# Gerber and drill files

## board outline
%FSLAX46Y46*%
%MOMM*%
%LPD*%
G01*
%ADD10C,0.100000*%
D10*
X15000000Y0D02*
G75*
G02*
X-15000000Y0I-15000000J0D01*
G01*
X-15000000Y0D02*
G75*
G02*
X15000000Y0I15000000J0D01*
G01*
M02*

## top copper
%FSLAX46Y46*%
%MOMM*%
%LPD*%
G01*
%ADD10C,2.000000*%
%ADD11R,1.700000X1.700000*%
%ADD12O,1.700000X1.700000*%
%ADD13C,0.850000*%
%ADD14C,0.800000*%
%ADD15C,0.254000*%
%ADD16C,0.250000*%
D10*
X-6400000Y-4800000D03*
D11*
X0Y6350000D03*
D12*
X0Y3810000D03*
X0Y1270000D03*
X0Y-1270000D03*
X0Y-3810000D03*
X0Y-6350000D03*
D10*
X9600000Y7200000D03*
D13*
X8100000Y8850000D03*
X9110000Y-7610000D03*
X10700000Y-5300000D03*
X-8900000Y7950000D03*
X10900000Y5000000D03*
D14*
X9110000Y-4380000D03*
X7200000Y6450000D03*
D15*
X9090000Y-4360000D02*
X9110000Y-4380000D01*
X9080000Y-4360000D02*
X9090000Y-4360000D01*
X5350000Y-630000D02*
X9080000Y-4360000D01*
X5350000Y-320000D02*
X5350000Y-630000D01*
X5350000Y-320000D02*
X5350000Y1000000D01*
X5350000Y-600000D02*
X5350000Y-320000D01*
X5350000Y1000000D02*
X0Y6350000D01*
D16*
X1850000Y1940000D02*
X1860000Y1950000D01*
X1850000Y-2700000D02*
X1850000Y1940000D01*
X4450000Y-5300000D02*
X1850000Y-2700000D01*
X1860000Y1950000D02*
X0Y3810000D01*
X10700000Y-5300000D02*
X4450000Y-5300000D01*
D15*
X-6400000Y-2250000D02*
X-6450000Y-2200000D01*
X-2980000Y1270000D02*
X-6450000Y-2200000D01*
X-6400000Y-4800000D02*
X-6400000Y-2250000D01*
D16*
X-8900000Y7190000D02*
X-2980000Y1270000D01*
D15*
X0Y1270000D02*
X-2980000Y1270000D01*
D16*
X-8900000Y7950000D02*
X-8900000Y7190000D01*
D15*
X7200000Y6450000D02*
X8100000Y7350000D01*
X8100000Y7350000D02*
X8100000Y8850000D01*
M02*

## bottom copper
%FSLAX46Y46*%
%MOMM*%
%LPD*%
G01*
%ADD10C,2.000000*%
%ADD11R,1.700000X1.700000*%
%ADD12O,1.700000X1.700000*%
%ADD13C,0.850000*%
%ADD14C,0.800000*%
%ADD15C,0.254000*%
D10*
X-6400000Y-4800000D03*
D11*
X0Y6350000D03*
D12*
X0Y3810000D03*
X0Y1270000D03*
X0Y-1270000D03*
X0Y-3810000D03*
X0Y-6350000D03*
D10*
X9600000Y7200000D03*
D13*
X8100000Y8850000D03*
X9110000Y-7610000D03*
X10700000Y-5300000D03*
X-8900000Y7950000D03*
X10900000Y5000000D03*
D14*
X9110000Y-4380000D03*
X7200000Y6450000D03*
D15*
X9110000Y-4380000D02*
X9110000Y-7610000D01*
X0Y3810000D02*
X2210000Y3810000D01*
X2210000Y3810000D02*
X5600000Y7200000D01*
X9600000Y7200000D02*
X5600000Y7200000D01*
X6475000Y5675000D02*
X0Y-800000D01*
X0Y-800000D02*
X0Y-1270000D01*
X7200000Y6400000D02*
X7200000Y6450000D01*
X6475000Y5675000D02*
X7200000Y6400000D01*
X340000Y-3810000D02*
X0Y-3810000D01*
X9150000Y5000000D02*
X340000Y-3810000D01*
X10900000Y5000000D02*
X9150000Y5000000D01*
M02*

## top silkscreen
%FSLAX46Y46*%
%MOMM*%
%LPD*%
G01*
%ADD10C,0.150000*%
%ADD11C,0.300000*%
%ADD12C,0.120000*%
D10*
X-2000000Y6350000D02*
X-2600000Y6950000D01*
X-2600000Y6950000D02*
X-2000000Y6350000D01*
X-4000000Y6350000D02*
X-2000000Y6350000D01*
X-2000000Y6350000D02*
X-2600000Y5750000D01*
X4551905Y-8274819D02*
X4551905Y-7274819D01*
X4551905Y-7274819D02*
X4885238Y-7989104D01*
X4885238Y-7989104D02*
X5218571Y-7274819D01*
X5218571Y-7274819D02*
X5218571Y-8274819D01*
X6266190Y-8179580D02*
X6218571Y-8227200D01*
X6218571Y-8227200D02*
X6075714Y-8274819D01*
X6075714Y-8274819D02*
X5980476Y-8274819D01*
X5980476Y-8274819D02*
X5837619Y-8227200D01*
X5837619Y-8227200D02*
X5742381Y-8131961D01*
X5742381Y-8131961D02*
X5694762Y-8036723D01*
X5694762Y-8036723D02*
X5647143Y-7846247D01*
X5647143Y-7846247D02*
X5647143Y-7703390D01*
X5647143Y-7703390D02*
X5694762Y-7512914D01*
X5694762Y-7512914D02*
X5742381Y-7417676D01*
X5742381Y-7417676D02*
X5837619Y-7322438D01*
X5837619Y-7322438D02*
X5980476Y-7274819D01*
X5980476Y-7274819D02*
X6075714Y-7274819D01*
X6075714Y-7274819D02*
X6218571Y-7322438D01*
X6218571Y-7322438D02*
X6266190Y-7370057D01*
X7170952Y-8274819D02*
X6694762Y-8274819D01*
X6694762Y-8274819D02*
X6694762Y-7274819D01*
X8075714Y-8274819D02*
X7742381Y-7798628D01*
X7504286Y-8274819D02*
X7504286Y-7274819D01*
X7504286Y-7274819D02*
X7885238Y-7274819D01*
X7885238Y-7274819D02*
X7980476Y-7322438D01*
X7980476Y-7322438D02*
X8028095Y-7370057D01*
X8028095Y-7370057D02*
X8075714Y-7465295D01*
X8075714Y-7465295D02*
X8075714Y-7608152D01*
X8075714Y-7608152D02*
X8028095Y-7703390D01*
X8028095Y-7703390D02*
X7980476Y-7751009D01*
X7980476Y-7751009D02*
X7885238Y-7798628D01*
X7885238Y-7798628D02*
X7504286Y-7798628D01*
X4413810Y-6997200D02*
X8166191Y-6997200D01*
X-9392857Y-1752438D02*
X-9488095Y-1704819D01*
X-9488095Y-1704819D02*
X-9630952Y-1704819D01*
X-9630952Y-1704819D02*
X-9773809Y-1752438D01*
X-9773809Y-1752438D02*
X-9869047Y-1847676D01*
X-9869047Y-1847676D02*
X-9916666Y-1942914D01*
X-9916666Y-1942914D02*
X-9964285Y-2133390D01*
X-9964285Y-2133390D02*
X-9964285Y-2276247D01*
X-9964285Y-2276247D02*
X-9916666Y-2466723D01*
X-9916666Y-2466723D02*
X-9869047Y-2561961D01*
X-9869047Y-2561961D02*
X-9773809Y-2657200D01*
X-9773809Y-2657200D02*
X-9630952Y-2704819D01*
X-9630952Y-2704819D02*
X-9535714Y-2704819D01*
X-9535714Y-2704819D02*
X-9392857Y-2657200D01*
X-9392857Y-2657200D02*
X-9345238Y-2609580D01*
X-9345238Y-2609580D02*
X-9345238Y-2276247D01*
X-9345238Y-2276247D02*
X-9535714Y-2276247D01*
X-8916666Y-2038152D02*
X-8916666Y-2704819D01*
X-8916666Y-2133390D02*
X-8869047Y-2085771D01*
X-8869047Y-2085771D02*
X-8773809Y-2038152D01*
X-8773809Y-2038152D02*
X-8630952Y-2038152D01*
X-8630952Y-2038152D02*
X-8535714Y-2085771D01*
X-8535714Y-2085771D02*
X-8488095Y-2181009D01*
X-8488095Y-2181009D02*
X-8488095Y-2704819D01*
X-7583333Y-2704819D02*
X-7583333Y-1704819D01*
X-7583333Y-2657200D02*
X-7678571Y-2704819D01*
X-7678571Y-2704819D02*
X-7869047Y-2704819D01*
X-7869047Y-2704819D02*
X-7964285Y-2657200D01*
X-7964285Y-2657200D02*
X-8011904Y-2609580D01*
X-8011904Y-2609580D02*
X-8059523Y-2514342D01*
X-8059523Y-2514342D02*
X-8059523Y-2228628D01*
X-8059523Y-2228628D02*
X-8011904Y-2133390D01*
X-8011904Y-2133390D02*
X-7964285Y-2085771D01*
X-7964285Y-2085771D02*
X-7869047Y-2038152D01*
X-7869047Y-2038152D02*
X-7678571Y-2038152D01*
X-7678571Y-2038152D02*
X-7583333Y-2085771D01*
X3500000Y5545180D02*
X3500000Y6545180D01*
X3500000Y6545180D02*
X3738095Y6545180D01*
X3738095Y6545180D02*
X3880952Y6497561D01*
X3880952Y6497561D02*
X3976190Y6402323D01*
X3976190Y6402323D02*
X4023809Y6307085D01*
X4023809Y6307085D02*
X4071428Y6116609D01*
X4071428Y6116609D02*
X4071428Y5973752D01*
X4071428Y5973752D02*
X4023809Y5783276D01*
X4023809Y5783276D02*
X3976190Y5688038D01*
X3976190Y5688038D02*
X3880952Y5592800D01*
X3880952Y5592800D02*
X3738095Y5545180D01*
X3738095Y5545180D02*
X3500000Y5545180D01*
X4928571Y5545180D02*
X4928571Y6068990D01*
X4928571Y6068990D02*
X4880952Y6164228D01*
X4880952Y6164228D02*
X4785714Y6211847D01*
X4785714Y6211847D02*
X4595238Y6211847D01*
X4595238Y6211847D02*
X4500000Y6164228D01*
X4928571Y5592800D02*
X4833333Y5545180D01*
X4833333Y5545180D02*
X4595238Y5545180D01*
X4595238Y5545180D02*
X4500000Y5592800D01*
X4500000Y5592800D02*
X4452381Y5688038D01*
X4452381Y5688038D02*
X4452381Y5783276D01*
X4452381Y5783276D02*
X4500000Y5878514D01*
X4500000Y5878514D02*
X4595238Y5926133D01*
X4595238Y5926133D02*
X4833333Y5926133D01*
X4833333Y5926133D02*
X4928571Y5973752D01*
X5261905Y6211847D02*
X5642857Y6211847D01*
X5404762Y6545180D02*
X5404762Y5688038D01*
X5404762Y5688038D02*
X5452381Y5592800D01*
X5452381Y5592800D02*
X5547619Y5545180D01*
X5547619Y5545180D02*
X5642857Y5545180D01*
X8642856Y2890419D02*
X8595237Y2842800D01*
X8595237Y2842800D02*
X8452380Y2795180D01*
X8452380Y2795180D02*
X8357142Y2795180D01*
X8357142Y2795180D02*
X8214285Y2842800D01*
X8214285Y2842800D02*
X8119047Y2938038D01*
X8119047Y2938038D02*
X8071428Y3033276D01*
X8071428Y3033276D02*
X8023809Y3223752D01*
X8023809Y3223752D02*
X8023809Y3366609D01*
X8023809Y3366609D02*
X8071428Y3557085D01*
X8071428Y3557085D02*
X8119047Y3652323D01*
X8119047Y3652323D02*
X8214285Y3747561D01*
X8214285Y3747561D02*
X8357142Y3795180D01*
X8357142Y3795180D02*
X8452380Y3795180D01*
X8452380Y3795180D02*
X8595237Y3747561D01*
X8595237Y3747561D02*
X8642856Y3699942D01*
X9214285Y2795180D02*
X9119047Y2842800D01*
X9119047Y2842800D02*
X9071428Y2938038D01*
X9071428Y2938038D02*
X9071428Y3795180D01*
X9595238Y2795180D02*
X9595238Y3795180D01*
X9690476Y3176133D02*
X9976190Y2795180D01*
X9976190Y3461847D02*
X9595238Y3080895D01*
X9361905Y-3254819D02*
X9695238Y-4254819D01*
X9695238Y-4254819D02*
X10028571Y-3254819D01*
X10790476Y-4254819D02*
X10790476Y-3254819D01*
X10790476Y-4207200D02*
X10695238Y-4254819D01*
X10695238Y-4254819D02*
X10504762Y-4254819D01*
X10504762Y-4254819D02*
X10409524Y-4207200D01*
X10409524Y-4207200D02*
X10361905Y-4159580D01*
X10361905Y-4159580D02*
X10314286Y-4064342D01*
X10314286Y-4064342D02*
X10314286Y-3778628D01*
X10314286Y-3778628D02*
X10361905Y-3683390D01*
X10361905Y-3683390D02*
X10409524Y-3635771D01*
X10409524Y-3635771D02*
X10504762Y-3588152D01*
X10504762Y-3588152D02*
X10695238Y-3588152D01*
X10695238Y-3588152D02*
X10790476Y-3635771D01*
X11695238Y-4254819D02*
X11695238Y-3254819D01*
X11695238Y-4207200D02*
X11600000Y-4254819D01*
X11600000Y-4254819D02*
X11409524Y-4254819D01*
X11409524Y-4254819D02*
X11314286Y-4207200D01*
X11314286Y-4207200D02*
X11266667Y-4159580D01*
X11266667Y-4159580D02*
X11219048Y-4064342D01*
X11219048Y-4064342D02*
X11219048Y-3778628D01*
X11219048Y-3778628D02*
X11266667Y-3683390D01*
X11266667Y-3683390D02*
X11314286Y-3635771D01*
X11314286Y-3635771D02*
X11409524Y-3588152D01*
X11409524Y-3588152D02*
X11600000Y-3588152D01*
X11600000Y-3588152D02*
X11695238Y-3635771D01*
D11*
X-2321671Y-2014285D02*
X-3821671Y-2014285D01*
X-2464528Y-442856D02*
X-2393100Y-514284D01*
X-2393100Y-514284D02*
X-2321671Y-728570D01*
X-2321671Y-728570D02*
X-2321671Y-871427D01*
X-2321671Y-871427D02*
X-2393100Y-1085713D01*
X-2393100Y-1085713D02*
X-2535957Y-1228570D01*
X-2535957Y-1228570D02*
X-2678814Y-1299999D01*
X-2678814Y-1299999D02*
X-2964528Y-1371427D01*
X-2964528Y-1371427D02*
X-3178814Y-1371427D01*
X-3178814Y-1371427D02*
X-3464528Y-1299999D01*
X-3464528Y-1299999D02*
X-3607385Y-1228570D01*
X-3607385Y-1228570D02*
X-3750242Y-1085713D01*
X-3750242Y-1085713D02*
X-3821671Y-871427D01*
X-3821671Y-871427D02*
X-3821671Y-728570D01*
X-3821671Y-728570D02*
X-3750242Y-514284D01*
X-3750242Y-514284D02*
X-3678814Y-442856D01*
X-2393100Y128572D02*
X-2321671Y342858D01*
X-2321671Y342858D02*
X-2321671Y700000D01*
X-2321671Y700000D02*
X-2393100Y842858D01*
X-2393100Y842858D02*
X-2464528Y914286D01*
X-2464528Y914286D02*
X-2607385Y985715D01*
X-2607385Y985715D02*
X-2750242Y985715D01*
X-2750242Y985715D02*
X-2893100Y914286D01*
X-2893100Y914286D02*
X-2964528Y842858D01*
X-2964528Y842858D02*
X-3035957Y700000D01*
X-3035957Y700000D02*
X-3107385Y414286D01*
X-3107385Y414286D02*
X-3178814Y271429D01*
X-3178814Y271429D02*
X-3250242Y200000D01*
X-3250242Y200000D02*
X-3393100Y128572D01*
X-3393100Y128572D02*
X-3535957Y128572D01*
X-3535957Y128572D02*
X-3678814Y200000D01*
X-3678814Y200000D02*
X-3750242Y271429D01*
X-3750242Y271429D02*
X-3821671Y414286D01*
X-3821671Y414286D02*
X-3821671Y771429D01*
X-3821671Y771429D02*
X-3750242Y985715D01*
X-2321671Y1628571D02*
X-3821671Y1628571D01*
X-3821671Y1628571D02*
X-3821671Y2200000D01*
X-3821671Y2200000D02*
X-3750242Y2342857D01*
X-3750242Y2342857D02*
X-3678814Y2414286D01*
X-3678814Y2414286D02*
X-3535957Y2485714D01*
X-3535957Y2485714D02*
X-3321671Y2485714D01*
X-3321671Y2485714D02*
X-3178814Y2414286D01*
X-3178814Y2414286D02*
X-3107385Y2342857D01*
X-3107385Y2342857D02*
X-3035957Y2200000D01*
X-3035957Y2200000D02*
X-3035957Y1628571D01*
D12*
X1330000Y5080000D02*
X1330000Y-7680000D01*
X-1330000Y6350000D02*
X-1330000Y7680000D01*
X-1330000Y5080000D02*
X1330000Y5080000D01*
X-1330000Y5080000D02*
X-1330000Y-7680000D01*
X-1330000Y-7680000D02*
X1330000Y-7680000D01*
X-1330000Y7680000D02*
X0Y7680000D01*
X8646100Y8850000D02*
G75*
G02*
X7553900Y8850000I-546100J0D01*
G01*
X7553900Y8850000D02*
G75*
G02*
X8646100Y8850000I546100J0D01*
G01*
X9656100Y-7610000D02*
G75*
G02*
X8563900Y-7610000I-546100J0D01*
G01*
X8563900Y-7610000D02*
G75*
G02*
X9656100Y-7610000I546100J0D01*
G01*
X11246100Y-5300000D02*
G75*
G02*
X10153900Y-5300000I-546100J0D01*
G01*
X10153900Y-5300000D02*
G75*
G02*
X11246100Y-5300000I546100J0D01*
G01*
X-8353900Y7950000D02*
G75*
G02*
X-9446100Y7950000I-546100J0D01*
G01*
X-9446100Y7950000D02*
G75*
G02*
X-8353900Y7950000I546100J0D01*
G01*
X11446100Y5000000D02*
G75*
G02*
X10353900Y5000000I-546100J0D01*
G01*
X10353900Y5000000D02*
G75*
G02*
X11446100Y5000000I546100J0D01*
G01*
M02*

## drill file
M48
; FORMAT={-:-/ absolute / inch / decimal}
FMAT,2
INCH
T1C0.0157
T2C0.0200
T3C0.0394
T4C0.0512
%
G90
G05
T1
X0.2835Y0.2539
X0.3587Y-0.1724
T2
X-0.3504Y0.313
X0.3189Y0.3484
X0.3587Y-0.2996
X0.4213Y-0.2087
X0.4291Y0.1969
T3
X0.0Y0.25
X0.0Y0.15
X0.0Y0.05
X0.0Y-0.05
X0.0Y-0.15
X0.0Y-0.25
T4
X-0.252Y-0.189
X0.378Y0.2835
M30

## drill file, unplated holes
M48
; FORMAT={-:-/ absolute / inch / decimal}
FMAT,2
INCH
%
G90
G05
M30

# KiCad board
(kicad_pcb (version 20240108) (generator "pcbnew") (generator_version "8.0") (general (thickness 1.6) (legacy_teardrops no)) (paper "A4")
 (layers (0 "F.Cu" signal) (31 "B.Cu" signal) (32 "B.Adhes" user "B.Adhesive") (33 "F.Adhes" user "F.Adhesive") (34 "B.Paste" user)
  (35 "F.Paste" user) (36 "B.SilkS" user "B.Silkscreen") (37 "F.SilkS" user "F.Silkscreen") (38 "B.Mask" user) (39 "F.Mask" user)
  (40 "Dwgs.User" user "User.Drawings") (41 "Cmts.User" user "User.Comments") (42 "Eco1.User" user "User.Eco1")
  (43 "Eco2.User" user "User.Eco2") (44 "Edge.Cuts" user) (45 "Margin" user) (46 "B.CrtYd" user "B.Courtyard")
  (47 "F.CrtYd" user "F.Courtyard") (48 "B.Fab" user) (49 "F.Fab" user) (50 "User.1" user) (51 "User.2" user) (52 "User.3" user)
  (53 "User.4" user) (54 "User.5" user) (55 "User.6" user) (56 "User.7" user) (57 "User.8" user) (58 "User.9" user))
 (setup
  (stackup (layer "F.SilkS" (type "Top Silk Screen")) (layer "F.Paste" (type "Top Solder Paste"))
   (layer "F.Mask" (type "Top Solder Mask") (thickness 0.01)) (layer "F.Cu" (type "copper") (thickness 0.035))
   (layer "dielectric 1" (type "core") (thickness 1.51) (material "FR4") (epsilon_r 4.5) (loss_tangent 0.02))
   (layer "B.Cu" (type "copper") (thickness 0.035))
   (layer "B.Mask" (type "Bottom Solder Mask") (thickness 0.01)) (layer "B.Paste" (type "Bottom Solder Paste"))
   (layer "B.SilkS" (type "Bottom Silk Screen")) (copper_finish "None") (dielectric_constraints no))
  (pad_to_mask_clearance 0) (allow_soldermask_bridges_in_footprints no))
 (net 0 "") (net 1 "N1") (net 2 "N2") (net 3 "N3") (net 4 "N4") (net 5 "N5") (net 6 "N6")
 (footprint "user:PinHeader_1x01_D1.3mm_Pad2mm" (layer "F.Cu") (at -6.4 4.8)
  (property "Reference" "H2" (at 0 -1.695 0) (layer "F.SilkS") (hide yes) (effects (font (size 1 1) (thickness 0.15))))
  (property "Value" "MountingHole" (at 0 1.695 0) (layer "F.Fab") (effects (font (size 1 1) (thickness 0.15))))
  (pad "1" thru_hole circle (at 0 0) (size 2 2) (drill 1.3) (layers "*.Cu" "*.Mask") (remove_unused_layers no) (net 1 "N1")))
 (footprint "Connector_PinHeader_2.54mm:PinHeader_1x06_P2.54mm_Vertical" (layer "F.Cu") (at 0 -6.35)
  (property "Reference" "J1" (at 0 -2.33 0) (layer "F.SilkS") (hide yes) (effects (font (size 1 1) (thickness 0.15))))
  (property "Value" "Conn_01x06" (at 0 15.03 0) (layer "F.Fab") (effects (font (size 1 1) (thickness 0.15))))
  (fp_line (start -1.33 -1.33) (end 0 -1.33) (stroke (width 0.12) (type solid)) (layer "F.SilkS"))
  (fp_line (start -1.33 0) (end -1.33 -1.33) (stroke (width 0.12) (type solid)) (layer "F.SilkS"))
  (fp_line (start -1.33 1.27) (end -1.33 14.03) (stroke (width 0.12) (type solid)) (layer "F.SilkS"))
  (fp_line (start -1.33 1.27) (end 1.33 1.27) (stroke (width 0.12) (type solid)) (layer "F.SilkS"))
  (fp_line (start -1.33 14.03) (end 1.33 14.03) (stroke (width 0.12) (type solid)) (layer "F.SilkS"))
  (fp_line (start 1.33 1.27) (end 1.33 14.03) (stroke (width 0.12) (type solid)) (layer "F.SilkS"))
  (pad "1" thru_hole rect (at 0 0) (size 1.7 1.7) (drill 1) (layers "*.Cu" "*.Mask") (remove_unused_layers no) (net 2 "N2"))
  (pad "2" thru_hole oval (at 0 2.54) (size 1.7 1.7) (drill 1) (layers "*.Cu" "*.Mask") (remove_unused_layers no) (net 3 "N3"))
  (pad "3" thru_hole oval (at 0 5.08) (size 1.7 1.7) (drill 1) (layers "*.Cu" "*.Mask") (remove_unused_layers no) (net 1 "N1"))
  (pad "4" thru_hole oval (at 0 7.62) (size 1.7 1.7) (drill 1) (layers "*.Cu" "*.Mask") (remove_unused_layers no) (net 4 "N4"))
  (pad "5" thru_hole oval (at 0 10.16) (size 1.7 1.7) (drill 1) (layers "*.Cu" "*.Mask") (remove_unused_layers no) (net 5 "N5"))
  (pad "6" thru_hole oval (at 0 12.7) (size 1.7 1.7) (drill 1) (layers "*.Cu" "*.Mask") (remove_unused_layers no) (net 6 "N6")))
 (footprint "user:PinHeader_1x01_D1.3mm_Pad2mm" (layer "F.Cu") (at 9.6 -7.2)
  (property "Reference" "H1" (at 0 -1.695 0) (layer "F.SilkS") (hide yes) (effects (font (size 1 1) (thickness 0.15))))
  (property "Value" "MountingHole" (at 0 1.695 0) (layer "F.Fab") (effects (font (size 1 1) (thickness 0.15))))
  (pad "1" thru_hole circle (at 0 0) (size 2 2) (drill 1.3) (layers "*.Cu" "*.Mask") (remove_unused_layers no) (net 3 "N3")))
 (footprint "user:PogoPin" (layer "F.Cu") (at 8.1 -8.85)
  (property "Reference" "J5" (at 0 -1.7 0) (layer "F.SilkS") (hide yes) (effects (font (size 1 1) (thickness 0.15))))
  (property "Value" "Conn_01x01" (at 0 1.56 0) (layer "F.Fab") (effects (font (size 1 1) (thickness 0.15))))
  (fp_circle (center 0 0) (end 0.5461 0) (stroke (width 0.12) (type solid)) (fill none) (layer "F.SilkS"))
  (pad "1" thru_hole circle (at 0 0) (size 0.85 0.85) (drill 0.508) (layers "*.Cu" "*.Mask") (remove_unused_layers no) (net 4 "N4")))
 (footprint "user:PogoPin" (layer "F.Cu") (at 9.11 7.61)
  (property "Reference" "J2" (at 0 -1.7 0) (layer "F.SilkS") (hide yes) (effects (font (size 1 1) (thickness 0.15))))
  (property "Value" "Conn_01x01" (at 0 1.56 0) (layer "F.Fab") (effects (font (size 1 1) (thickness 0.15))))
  (fp_circle (center 0 0) (end 0.5461 0) (stroke (width 0.12) (type solid)) (fill none) (layer "F.SilkS"))
  (pad "1" thru_hole circle (at 0 0) (size 0.85 0.85) (drill 0.508) (layers "*.Cu" "*.Mask") (remove_unused_layers no) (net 2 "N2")))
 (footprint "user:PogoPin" (layer "F.Cu") (at 10.7 5.3)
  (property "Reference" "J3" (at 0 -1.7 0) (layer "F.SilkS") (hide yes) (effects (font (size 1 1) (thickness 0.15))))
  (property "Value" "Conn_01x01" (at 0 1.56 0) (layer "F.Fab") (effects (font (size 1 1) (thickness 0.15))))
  (fp_circle (center 0 0) (end 0.5461 0) (stroke (width 0.12) (type solid)) (fill none) (layer "F.SilkS"))
  (pad "1" thru_hole circle (at 0 0) (size 0.85 0.85) (drill 0.508) (layers "*.Cu" "*.Mask") (remove_unused_layers no) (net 3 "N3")))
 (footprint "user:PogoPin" (layer "F.Cu") (at -8.9 -7.95)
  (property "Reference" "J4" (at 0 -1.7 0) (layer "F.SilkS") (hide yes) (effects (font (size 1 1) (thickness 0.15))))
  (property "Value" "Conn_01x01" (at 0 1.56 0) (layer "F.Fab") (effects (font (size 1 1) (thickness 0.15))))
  (fp_circle (center 0 0) (end 0.5461 0) (stroke (width 0.12) (type solid)) (fill none) (layer "F.SilkS"))
  (pad "1" thru_hole circle (at 0 0) (size 0.85 0.85) (drill 0.508) (layers "*.Cu" "*.Mask") (remove_unused_layers no) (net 1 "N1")))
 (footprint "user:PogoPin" (layer "F.Cu") (at 10.9 -5)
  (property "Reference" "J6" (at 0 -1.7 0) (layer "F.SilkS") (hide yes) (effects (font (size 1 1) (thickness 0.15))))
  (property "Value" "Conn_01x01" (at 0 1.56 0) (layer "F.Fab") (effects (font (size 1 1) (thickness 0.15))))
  (fp_circle (center 0 0) (end 0.5461 0) (stroke (width 0.12) (type solid)) (fill none) (layer "F.SilkS"))
  (pad "1" thru_hole circle (at 0 0) (size 0.85 0.85) (drill 0.508) (layers "*.Cu" "*.Mask") (remove_unused_layers no) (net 5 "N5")))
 (gr_line (start -2 -6.35) (end -2.6 -6.95) (stroke (width 0.15) (type solid)) (layer "F.SilkS"))
 (gr_line (start -2.6 -6.95) (end -2 -6.35) (stroke (width 0.15) (type solid)) (layer "F.SilkS"))
 (gr_line (start -4 -6.35) (end -2 -6.35) (stroke (width 0.15) (type solid)) (layer "F.SilkS"))
 (gr_line (start -2 -6.35) (end -2.6 -5.75) (stroke (width 0.15) (type solid)) (layer "F.SilkS"))
 (gr_circle (center 0 0) (end 15 0) (stroke (width 0.1) (type solid)) (fill none) (layer "Edge.Cuts"))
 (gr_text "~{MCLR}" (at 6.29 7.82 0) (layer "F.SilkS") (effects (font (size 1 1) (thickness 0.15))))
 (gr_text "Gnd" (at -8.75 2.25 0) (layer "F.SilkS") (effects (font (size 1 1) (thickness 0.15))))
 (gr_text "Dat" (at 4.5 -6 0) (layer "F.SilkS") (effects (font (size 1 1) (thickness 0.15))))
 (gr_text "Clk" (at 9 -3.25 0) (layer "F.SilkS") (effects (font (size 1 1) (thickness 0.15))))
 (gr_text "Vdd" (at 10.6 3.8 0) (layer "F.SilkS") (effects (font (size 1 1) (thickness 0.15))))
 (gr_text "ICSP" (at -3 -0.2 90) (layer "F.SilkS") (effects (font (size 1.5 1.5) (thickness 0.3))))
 (segment (start 5.35 0.63) (end 9.08 4.36) (width 0.254) (layer "F.Cu") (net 2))
 (segment (start 9.08 4.36) (end 9.09 4.36) (width 0.254) (layer "F.Cu") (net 2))
 (segment (start 5.35 0.6) (end 5.35 0.32) (width 0.254) (layer "F.Cu") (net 2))
 (segment (start 9.09 4.36) (end 9.11 4.38) (width 0.254) (layer "F.Cu") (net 2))
 (segment (start 5.35 0.32) (end 5.35 -1) (width 0.254) (layer "F.Cu") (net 2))
 (segment (start 5.35 -1) (end 0 -6.35) (width 0.254) (layer "F.Cu") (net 2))
 (segment (start 5.35 0.32) (end 5.35 0.63) (width 0.254) (layer "F.Cu") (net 2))
 (via (at 9.11 4.38) (size 0.8) (drill 0.4) (layers "F.Cu" "B.Cu") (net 2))
 (segment (start 9.11 4.38) (end 9.11 7.61) (width 0.254) (layer "B.Cu") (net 2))
 (segment (start 1.85 -1.94) (end 1.86 -1.95) (width 0.25) (layer "F.Cu") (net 3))
 (segment (start 1.85 2.7) (end 1.85 -1.94) (width 0.25) (layer "F.Cu") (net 3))
 (segment (start 4.45 5.3) (end 1.85 2.7) (width 0.25) (layer "F.Cu") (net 3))
 (segment (start 1.86 -1.95) (end 0 -3.81) (width 0.25) (layer "F.Cu") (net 3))
 (segment (start 10.7 5.3) (end 4.45 5.3) (width 0.25) (layer "F.Cu") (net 3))
 (segment (start 0 -3.81) (end 2.21 -3.81) (width 0.254) (layer "B.Cu") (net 3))
 (segment (start 2.21 -3.81) (end 5.6 -7.2) (width 0.254) (layer "B.Cu") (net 3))
 (segment (start 9.6 -7.2) (end 5.6 -7.2) (width 0.254) (layer "B.Cu") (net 3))
 (segment (start -6.4 2.25) (end -6.45 2.2) (width 0.254) (layer "F.Cu") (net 1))
 (segment (start -2.98 -1.27) (end -6.45 2.2) (width 0.254) (layer "F.Cu") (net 1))
 (segment (start -6.4 4.8) (end -6.4 2.25) (width 0.254) (layer "F.Cu") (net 1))
 (segment (start -8.9 -7.19) (end -2.98 -1.27) (width 0.25) (layer "F.Cu") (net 1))
 (segment (start 0 -1.27) (end -2.98 -1.27) (width 0.254) (layer "F.Cu") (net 1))
 (segment (start -8.9 -7.95) (end -8.9 -7.19) (width 0.25) (layer "F.Cu") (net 1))
 (segment (start 7.2 -6.45) (end 8.1 -7.35) (width 0.254) (layer "F.Cu") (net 4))
 (segment (start 8.1 -7.35) (end 8.1 -8.85) (width 0.254) (layer "F.Cu") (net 4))
 (via (at 7.2 -6.45) (size 0.8) (drill 0.4) (layers "F.Cu" "B.Cu") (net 4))
 (segment (start 6.475 -5.675) (end 0 0.8) (width 0.254) (layer "B.Cu") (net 4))
 (segment (start 0 0.8) (end 0 1.27) (width 0.254) (layer "B.Cu") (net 4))
 (segment (start 7.2 -6.4) (end 7.2 -6.45) (width 0.254) (layer "B.Cu") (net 4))
 (segment (start 6.475 -5.675) (end 7.2 -6.4) (width 0.254) (layer "B.Cu") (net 4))
 (segment (start 0.34 3.81) (end 0 3.81) (width 0.254) (layer "B.Cu") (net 5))
 (segment (start 9.15 -5) (end 0.34 3.81) (width 0.254) (layer "B.Cu") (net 5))
 (segment (start 10.9 -5) (end 9.15 -5) (width 0.254) (layer "B.Cu") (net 5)))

